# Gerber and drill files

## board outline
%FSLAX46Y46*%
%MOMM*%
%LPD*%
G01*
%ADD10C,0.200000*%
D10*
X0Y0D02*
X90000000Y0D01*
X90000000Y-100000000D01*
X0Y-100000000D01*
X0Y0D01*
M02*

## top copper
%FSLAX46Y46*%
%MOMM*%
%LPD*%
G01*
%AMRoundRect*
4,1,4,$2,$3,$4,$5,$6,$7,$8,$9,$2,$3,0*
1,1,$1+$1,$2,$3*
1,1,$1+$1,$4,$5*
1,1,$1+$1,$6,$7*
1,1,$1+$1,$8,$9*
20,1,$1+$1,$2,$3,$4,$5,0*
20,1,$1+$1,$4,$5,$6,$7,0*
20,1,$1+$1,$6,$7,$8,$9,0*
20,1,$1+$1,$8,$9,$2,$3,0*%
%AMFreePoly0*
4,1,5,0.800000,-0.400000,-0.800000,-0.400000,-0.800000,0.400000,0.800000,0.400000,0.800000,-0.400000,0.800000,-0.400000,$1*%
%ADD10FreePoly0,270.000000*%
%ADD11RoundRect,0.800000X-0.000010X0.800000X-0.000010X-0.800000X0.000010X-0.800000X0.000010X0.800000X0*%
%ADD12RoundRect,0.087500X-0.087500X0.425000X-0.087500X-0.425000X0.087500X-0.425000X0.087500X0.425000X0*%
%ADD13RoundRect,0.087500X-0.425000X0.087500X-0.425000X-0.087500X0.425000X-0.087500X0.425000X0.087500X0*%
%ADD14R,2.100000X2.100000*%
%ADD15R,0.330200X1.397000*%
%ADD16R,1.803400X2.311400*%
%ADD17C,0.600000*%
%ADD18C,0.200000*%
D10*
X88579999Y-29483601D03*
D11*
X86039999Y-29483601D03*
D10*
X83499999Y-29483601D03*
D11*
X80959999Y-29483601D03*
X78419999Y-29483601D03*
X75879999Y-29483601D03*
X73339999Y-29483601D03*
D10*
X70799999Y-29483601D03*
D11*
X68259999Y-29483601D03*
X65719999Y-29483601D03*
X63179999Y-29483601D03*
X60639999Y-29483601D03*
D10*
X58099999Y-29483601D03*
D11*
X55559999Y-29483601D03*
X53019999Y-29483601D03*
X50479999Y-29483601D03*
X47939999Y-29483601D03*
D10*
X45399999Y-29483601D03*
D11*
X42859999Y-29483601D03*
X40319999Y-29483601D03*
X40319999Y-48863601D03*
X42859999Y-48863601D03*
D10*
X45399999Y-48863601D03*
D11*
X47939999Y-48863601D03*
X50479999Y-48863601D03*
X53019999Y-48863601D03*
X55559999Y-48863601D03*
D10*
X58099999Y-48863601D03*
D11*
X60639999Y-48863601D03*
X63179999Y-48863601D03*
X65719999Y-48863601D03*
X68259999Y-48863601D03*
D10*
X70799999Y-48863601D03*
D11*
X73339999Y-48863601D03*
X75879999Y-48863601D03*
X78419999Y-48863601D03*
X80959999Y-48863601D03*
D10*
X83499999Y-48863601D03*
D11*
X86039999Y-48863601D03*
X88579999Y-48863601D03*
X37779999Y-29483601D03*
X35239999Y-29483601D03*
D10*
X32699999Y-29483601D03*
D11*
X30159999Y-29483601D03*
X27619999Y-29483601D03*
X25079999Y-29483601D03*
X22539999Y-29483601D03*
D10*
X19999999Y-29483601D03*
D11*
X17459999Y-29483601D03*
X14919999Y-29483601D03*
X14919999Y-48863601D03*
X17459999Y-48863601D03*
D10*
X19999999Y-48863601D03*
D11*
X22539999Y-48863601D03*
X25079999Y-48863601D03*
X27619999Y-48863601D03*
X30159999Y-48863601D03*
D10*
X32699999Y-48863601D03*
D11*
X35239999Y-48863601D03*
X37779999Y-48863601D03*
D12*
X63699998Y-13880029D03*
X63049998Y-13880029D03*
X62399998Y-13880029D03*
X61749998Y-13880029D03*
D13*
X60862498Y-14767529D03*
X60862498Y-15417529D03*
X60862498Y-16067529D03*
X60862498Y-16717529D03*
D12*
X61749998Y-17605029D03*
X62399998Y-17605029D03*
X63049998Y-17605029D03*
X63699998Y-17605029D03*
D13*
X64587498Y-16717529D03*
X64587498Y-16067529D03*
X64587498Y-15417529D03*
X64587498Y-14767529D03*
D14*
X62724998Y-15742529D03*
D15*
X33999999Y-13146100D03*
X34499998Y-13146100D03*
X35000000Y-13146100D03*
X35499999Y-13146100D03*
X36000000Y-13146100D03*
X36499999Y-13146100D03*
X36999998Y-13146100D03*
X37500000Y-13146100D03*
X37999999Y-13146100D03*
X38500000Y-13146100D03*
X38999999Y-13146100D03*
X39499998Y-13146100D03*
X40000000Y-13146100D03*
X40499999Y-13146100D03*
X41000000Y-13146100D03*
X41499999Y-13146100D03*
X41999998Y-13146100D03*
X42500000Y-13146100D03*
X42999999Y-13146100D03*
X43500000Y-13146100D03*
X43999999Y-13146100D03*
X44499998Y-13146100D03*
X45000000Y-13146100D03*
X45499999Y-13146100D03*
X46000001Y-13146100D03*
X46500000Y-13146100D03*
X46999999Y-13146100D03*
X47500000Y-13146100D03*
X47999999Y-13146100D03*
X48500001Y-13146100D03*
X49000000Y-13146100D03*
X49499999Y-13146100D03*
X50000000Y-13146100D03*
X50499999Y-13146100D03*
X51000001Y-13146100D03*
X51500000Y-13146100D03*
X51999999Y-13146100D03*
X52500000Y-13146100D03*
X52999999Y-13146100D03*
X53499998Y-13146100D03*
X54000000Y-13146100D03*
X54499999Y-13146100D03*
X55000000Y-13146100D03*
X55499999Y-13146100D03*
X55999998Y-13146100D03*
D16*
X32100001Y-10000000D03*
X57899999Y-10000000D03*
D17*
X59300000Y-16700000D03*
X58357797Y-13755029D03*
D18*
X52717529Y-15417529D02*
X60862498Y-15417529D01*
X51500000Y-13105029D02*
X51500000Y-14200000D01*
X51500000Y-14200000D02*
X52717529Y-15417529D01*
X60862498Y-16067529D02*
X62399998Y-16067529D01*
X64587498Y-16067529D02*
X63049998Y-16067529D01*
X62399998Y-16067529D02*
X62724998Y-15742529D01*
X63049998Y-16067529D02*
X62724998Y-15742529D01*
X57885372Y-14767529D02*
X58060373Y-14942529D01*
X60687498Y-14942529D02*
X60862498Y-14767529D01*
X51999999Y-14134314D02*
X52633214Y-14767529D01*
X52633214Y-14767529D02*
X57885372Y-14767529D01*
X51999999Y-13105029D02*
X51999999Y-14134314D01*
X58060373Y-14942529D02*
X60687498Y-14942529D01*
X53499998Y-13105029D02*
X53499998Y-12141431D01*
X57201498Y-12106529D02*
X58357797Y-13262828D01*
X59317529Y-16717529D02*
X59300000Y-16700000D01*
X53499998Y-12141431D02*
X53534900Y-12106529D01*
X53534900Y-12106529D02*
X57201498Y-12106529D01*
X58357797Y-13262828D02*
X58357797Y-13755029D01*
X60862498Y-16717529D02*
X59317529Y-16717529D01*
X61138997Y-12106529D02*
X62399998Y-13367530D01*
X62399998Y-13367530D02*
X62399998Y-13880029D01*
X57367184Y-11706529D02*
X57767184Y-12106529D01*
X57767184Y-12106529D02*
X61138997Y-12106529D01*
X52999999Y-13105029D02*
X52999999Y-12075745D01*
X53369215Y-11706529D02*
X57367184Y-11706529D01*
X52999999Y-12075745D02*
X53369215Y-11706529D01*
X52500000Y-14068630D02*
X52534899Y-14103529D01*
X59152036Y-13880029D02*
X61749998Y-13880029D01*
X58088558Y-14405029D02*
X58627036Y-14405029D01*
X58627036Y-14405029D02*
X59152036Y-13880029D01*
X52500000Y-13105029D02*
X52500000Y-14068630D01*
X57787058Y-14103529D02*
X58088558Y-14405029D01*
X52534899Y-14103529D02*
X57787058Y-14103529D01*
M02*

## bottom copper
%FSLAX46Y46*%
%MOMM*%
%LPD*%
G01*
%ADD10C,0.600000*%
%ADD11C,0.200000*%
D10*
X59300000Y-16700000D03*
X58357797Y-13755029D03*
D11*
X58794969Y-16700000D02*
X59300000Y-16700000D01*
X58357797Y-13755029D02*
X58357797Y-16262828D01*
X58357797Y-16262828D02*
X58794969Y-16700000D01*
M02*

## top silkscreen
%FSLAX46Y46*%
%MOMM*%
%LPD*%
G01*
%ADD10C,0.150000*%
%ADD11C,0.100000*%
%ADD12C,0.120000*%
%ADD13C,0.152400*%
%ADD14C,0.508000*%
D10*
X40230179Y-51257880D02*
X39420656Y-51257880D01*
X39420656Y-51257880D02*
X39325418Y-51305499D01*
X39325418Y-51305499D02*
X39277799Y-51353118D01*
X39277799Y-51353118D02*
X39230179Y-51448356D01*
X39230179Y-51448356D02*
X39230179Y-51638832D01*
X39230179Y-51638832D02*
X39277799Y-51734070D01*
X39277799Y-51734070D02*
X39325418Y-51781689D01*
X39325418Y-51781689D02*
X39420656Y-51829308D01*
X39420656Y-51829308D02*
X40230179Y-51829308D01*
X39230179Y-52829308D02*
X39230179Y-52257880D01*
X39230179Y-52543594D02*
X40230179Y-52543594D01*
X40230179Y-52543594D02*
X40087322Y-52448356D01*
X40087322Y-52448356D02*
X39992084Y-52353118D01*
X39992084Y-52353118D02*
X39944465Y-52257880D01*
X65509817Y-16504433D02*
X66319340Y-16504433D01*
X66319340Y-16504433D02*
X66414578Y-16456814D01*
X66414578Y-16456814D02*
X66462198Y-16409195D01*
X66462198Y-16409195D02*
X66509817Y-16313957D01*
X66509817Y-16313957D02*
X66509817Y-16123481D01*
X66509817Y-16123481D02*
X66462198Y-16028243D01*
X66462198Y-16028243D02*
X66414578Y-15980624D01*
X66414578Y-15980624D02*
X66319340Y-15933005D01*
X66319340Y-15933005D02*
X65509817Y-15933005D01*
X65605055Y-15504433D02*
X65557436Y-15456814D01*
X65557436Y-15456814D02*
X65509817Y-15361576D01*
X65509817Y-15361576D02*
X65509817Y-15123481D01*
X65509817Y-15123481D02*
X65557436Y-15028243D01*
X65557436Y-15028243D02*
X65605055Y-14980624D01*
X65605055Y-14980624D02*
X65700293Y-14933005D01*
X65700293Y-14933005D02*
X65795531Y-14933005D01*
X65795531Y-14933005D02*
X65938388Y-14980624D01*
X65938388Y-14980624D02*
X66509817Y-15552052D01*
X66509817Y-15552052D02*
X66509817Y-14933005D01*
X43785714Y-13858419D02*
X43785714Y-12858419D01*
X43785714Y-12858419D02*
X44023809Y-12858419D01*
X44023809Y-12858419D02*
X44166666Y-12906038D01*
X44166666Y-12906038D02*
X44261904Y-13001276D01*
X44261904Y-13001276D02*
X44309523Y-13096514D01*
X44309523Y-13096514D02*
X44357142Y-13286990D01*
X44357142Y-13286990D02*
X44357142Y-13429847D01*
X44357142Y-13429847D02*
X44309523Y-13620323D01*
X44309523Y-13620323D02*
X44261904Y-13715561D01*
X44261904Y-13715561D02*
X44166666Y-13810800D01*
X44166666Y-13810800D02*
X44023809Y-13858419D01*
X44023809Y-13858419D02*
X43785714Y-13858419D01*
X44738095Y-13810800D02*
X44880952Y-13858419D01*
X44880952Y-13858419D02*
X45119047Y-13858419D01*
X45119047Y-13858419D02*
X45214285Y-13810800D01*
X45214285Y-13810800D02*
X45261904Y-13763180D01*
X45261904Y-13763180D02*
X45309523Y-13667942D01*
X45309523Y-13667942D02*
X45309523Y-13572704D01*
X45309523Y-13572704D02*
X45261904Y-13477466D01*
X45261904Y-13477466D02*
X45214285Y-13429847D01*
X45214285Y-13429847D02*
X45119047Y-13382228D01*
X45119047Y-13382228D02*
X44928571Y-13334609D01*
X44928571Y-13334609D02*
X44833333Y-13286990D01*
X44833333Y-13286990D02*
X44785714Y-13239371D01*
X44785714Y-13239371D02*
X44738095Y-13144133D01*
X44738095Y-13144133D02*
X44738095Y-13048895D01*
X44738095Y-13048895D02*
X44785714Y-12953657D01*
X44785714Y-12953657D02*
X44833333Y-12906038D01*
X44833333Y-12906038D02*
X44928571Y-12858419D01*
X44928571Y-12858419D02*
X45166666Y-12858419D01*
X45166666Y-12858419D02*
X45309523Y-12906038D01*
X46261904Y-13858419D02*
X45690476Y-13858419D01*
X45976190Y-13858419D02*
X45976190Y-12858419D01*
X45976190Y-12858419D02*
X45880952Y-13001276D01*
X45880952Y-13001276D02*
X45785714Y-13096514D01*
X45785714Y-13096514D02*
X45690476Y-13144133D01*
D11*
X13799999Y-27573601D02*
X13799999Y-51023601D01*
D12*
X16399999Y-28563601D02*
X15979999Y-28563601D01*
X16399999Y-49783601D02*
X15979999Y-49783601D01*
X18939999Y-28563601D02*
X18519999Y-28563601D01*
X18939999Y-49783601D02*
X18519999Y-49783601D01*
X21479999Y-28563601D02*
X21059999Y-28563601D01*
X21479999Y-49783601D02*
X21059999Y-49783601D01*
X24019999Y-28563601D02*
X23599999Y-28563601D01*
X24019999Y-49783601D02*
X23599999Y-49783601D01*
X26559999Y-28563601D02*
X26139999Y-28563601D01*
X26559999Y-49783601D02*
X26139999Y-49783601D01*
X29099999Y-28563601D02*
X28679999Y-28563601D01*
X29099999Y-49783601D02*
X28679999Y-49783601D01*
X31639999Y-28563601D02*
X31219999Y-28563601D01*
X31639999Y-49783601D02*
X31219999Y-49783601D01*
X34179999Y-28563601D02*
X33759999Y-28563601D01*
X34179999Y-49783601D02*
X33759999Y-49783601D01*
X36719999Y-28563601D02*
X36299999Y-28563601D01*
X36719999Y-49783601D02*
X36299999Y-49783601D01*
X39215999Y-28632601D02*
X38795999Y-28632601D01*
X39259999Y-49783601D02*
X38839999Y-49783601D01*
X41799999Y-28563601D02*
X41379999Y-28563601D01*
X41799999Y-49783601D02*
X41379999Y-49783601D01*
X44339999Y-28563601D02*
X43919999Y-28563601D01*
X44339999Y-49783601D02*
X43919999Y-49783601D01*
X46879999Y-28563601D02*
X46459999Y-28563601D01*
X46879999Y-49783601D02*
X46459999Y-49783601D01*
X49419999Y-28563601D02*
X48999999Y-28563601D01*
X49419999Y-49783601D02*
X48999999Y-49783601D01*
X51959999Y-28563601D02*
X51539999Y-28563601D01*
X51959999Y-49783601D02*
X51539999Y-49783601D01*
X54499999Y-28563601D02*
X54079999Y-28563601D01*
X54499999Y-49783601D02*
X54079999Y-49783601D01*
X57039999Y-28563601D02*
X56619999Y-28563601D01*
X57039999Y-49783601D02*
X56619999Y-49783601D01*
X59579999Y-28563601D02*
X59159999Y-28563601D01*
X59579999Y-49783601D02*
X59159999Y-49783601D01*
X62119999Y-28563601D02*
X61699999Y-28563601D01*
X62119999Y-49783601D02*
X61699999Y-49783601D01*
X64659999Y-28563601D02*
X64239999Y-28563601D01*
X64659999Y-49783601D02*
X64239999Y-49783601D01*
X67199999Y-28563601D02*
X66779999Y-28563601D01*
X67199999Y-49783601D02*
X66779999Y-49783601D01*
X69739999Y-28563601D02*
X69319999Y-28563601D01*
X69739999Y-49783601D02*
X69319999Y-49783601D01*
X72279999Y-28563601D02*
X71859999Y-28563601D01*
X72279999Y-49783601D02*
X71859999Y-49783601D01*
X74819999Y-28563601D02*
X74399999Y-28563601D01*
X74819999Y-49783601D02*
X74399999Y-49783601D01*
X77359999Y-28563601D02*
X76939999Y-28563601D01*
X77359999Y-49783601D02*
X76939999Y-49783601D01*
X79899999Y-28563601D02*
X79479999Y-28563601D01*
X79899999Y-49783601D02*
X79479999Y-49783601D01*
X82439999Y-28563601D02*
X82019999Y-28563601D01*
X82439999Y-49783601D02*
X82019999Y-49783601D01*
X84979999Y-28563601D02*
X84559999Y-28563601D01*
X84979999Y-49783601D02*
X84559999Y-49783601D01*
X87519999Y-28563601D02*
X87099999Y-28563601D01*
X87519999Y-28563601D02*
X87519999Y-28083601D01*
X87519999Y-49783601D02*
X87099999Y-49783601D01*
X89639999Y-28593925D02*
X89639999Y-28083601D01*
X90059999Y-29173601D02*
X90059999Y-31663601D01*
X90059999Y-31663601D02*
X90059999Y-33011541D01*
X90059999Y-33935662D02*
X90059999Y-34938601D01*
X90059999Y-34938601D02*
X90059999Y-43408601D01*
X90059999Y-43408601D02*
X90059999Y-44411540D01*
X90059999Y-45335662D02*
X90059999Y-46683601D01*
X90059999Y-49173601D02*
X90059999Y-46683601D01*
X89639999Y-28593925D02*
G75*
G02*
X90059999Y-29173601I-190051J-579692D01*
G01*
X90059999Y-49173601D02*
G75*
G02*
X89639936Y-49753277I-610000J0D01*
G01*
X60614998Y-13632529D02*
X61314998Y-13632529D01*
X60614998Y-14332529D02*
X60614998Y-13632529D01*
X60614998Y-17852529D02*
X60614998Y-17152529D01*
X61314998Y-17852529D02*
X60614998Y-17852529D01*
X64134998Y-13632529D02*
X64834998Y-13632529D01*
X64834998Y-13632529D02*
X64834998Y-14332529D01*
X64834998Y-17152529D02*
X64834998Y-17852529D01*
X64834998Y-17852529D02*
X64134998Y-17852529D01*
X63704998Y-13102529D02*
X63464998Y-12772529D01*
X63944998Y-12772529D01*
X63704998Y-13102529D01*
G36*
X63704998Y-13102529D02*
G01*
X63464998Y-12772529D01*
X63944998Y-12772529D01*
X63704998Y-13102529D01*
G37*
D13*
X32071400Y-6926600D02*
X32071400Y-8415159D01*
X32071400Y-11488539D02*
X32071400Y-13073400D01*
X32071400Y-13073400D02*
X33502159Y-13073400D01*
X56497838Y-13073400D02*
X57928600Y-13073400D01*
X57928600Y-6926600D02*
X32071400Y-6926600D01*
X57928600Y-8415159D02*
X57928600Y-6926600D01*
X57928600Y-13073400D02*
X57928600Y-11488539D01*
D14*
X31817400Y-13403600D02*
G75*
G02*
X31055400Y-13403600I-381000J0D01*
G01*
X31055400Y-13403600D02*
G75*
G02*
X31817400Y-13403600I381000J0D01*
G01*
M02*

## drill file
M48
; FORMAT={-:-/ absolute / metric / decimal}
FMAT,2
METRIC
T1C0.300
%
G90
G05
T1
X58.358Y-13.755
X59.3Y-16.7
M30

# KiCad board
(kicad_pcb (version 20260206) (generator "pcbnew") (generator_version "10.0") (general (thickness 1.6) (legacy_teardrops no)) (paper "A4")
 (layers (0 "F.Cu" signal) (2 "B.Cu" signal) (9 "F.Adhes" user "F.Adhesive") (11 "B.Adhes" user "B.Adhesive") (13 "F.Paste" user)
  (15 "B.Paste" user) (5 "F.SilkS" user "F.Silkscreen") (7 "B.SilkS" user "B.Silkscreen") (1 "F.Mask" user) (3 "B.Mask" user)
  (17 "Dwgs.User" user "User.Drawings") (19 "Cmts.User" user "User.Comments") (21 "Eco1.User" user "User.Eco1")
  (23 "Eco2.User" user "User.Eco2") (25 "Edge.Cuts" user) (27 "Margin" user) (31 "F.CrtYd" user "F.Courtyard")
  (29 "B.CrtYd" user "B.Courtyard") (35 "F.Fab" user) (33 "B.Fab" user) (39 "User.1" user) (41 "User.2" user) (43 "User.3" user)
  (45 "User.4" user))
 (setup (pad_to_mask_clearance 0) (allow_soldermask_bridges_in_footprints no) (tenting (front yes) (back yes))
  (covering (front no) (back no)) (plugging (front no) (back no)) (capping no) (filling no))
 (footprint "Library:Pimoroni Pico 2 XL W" (layer "F.Cu") (at 64.449999 39.173601 -90)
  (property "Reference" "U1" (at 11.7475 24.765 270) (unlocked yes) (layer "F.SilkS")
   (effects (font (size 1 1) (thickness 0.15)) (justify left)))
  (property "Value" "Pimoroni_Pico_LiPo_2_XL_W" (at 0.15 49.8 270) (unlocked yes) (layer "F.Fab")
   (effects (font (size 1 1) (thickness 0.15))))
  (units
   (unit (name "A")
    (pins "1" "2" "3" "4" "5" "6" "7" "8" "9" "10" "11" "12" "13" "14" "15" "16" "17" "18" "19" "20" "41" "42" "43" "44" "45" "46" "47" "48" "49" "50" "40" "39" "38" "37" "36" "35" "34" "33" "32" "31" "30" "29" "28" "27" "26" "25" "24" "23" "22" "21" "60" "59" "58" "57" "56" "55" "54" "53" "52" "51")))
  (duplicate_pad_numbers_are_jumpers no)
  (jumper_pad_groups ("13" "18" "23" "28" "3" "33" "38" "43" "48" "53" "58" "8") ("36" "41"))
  (fp_line (start -11.6 50.65) (end 11.85 50.65) (stroke (width 0.1) (type default)) (layer "F.SilkS"))
  (fp_line (start -10.61 48.05) (end -10.61 48.47) (stroke (width 0.12) (type solid)) (layer "F.SilkS"))
  (fp_line (start 10.61 48.05) (end 10.61 48.47) (stroke (width 0.12) (type solid)) (layer "F.SilkS"))
  (fp_line (start -10.61 45.51) (end -10.61 45.93) (stroke (width 0.12) (type solid)) (layer "F.SilkS"))
  (fp_line (start 10.61 45.51) (end 10.61 45.93) (stroke (width 0.12) (type solid)) (layer "F.SilkS"))
  (fp_line (start -10.61 42.97) (end -10.61 43.39) (stroke (width 0.12) (type solid)) (layer "F.SilkS"))
  (fp_line (start 10.61 42.97) (end 10.61 43.39) (stroke (width 0.12) (type solid)) (layer "F.SilkS"))
  (fp_line (start -10.61 40.43) (end -10.61 40.85) (stroke (width 0.12) (type solid)) (layer "F.SilkS"))
  (fp_line (start 10.61 40.43) (end 10.61 40.85) (stroke (width 0.12) (type solid)) (layer "F.SilkS"))
  (fp_line (start -10.61 37.89) (end -10.61 38.31) (stroke (width 0.12) (type solid)) (layer "F.SilkS"))
  (fp_line (start 10.61 37.89) (end 10.61 38.31) (stroke (width 0.12) (type solid)) (layer "F.SilkS"))
  (fp_line (start -10.61 35.35) (end -10.61 35.77) (stroke (width 0.12) (type solid)) (layer "F.SilkS"))
  (fp_line (start 10.61 35.35) (end 10.61 35.77) (stroke (width 0.12) (type solid)) (layer "F.SilkS"))
  (fp_line (start -10.61 32.81) (end -10.61 33.23) (stroke (width 0.12) (type solid)) (layer "F.SilkS"))
  (fp_line (start 10.61 32.81) (end 10.61 33.23) (stroke (width 0.12) (type solid)) (layer "F.SilkS"))
  (fp_line (start -10.61 30.27) (end -10.61 30.69) (stroke (width 0.12) (type solid)) (layer "F.SilkS"))
  (fp_line (start 10.61 30.27) (end 10.61 30.69) (stroke (width 0.12) (type solid)) (layer "F.SilkS"))
  (fp_line (start -10.61 27.73) (end -10.61 28.15) (stroke (width 0.12) (type solid)) (layer "F.SilkS"))
  (fp_line (start 10.61 27.73) (end 10.61 28.15) (stroke (width 0.12) (type solid)) (layer "F.SilkS"))
  (fp_line (start -10.541 25.234) (end -10.541 25.654) (stroke (width 0.12) (type solid)) (layer "F.SilkS"))
  (fp_line (start 10.61 25.19) (end 10.61 25.61) (stroke (width 0.12) (type solid)) (layer "F.SilkS"))
  (fp_line (start -10.61 22.65) (end -10.61 23.07) (stroke (width 0.12) (type solid)) (layer "F.SilkS"))
  (fp_line (start 10.61 22.65) (end 10.61 23.07) (stroke (width 0.12) (type solid)) (layer "F.SilkS"))
  (fp_line (start -10.61 20.11) (end -10.61 20.53) (stroke (width 0.12) (type solid)) (layer "F.SilkS"))
  (fp_line (start 10.61 20.11) (end 10.61 20.53) (stroke (width 0.12) (type solid)) (layer "F.SilkS"))
  (fp_line (start -10.61 17.57) (end -10.61 17.99) (stroke (width 0.12) (type solid)) (layer "F.SilkS"))
  (fp_line (start 10.61 17.57) (end 10.61 17.99) (stroke (width 0.12) (type solid)) (layer "F.SilkS"))
  (fp_line (start -10.61 15.03) (end -10.61 15.45) (stroke (width 0.12) (type solid)) (layer "F.SilkS"))
  (fp_line (start 10.61 15.03) (end 10.61 15.45) (stroke (width 0.12) (type solid)) (layer "F.SilkS"))
  (fp_line (start -10.61 12.49) (end -10.61 12.91) (stroke (width 0.12) (type solid)) (layer "F.SilkS"))
  (fp_line (start 10.61 12.49) (end 10.61 12.91) (stroke (width 0.12) (type solid)) (layer "F.SilkS"))
  (fp_line (start -10.61 9.95) (end -10.61 10.37) (stroke (width 0.12) (type solid)) (layer "F.SilkS"))
  (fp_line (start 10.61 9.95) (end 10.61 10.37) (stroke (width 0.12) (type solid)) (layer "F.SilkS"))
  (fp_line (start -10.61 7.41) (end -10.61 7.83) (stroke (width 0.12) (type solid)) (layer "F.SilkS"))
  (fp_line (start 10.61 7.41) (end 10.61 7.83) (stroke (width 0.12) (type solid)) (layer "F.SilkS"))
  (fp_line (start -10.61 4.87) (end -10.61 5.29) (stroke (width 0.12) (type solid)) (layer "F.SilkS"))
  (fp_line (start 10.61 4.87) (end 10.61 5.29) (stroke (width 0.12) (type solid)) (layer "F.SilkS"))
  (fp_line (start -10.61 2.33) (end -10.61 2.75) (stroke (width 0.12) (type solid)) (layer "F.SilkS"))
  (fp_line (start 10.61 2.33) (end 10.61 2.75) (stroke (width 0.12) (type solid)) (layer "F.SilkS"))
  (fp_line (start -10.61 -0.21) (end -10.61 0.21) (stroke (width 0.12) (type solid)) (layer "F.SilkS"))
  (fp_line (start 10.61 -0.21) (end 10.61 0.21) (stroke (width 0.12) (type solid)) (layer "F.SilkS"))
  (fp_line (start -10.61 -2.75) (end -10.61 -2.33) (stroke (width 0.12) (type solid)) (layer "F.SilkS"))
  (fp_line (start 10.61 -2.75) (end 10.61 -2.33) (stroke (width 0.12) (type solid)) (layer "F.SilkS"))
  (fp_line (start -10.61 -5.29) (end -10.61 -4.87) (stroke (width 0.12) (type solid)) (layer "F.SilkS"))
  (fp_line (start 10.61 -5.29) (end 10.61 -4.87) (stroke (width 0.12) (type solid)) (layer "F.SilkS"))
  (fp_line (start -10.61 -7.83) (end -10.61 -7.41) (stroke (width 0.12) (type solid)) (layer "F.SilkS"))
  (fp_line (start 10.61 -7.83) (end 10.61 -7.41) (stroke (width 0.12) (type solid)) (layer "F.SilkS"))
  (fp_line (start -10.61 -10.37) (end -10.61 -9.95) (stroke (width 0.12) (type solid)) (layer "F.SilkS"))
  (fp_line (start 10.61 -10.37) (end 10.61 -9.95) (stroke (width 0.12) (type solid)) (layer "F.SilkS"))
  (fp_line (start -10.61 -12.91) (end -10.61 -12.49) (stroke (width 0.12) (type solid)) (layer "F.SilkS"))
  (fp_line (start 10.61 -12.91) (end 10.61 -12.49) (stroke (width 0.12) (type solid)) (layer "F.SilkS"))
  (fp_line (start -10.61 -15.45) (end -10.61 -15.03) (stroke (width 0.12) (type solid)) (layer "F.SilkS"))
  (fp_line (start 10.61 -15.45) (end 10.61 -15.03) (stroke (width 0.12) (type solid)) (layer "F.SilkS"))
  (fp_line (start -10.61 -17.99) (end -10.61 -17.57) (stroke (width 0.12) (type solid)) (layer "F.SilkS"))
  (fp_line (start 10.61 -17.99) (end 10.61 -17.57) (stroke (width 0.12) (type solid)) (layer "F.SilkS"))
  (fp_line (start -10.61 -20.53) (end -10.61 -20.11) (stroke (width 0.12) (type solid)) (layer "F.SilkS"))
  (fp_line (start 10.61 -20.53) (end 10.61 -20.11) (stroke (width 0.12) (type solid)) (layer "F.SilkS"))
  (fp_line (start -10.61 -23.07) (end -10.61 -22.65) (stroke (width 0.12) (type solid)) (layer "F.SilkS"))
  (fp_line (start -10.61 -23.07) (end -11.09 -23.07) (stroke (width 0.12) (type solid)) (layer "F.SilkS"))
  (fp_line (start 10.61 -23.07) (end 10.61 -22.65) (stroke (width 0.12) (type solid)) (layer "F.SilkS"))
  (fp_line (start -10.579676 -25.19) (end -11.09 -25.19) (stroke (width 0.12) (type solid)) (layer "F.SilkS"))
  (fp_line (start -10 -25.61) (end -7.51 -25.61) (stroke (width 0.12) (type solid)) (layer "F.SilkS"))
  (fp_line (start -7.51 -25.61) (end -6.16206 -25.61) (stroke (width 0.12) (type solid)) (layer "F.SilkS"))
  (fp_line (start -5.237939 -25.61) (end -4.235 -25.61) (stroke (width 0.12) (type solid)) (layer "F.SilkS"))
  (fp_line (start -4.235 -25.61) (end 4.235 -25.61) (stroke (width 0.12) (type solid)) (layer "F.SilkS"))
  (fp_line (start 4.235 -25.61) (end 5.237939 -25.61) (stroke (width 0.12) (type solid)) (layer "F.SilkS"))
  (fp_line (start 6.162061 -25.61) (end 7.51 -25.61) (stroke (width 0.12) (type solid)) (layer "F.SilkS"))
  (fp_line (start 10 -25.61) (end 7.51 -25.61) (stroke (width 0.12) (type solid)) (layer "F.SilkS"))
  (fp_arc (start -10.579676 -25.19) (mid -10.357938 -25.493944) (end -10 -25.61) (stroke (width 0.12) (type solid)) (layer "F.SilkS"))
  (fp_arc (start 10 -25.61) (mid 10.357937 -25.493944) (end 10.579676 -25.189937) (stroke (width 0.12) (type solid)) (layer "F.SilkS"))
  (pad "" smd rect (at -8.89 -24.13 270) (size 3.8 2.2) (drill (offset -0.8 0)) (layers "F.Paste"))
  (pad "" smd rect (at -8.89 -21.59 270) (size 3.8 2.2) (drill (offset -0.8 0)) (layers "F.Paste"))
  (pad "" smd rect (at -8.89 -19.05 270) (size 3.8 2.2) (drill (offset -0.8 0)) (layers "F.Paste"))
  (pad "" smd rect (at -8.89 -16.51 270) (size 3.8 2.2) (drill (offset -0.8 0)) (layers "F.Paste"))
  (pad "" smd rect (at -8.89 -13.97 270) (size 3.8 2.2) (drill (offset -0.8 0)) (layers "F.Paste"))
  (pad "" smd rect (at -8.89 -11.43 270) (size 3.8 2.2) (drill (offset -0.8 0)) (layers "F.Paste"))
  (pad "" smd rect (at -8.89 -8.89 270) (size 3.8 2.2) (drill (offset -0.8 0)) (layers "F.Paste"))
  (pad "" smd rect (at -8.89 -6.35 270) (size 3.8 2.2) (drill (offset -0.8 0)) (layers "F.Paste"))
  (pad "" smd rect (at -8.89 -3.81 270) (size 3.8 2.2) (drill (offset -0.8 0)) (layers "F.Paste"))
  (pad "" smd rect (at -8.89 -1.27 270) (size 3.8 2.2) (drill (offset -0.8 0)) (layers "F.Paste"))
  (pad "" smd rect (at -8.89 1.27 270) (size 3.8 2.2) (drill (offset -0.8 0)) (layers "F.Paste"))
  (pad "" smd rect (at -8.89 3.81 270) (size 3.8 2.2) (drill (offset -0.8 0)) (layers "F.Paste"))
  (pad "" smd rect (at -8.89 6.35 270) (size 3.8 2.2) (drill (offset -0.8 0)) (layers "F.Paste"))
  (pad "" smd rect (at -8.89 8.89 270) (size 3.8 2.2) (drill (offset -0.8 0)) (layers "F.Paste"))
  (pad "" smd rect (at -8.89 11.43 270) (size 3.8 2.2) (drill (offset -0.8 0)) (layers "F.Paste"))
  (pad "" smd rect (at -8.89 13.97 270) (size 3.8 2.2) (drill (offset -0.8 0)) (layers "F.Paste"))
  (pad "" smd rect (at -8.89 16.51 270) (size 3.8 2.2) (drill (offset -0.8 0)) (layers "F.Paste"))
  (pad "" smd rect (at -8.89 19.05 270) (size 3.8 2.2) (drill (offset -0.8 0)) (layers "F.Paste"))
  (pad "" smd rect (at -8.89 21.59 270) (size 3.8 2.2) (drill (offset -0.8 0)) (layers "F.Paste"))
  (pad "" smd rect (at -8.89 24.13 270) (size 3.8 2.2) (drill (offset -0.8 0)) (layers "F.Paste"))
  (pad "" smd rect (at -8.89 26.67 270) (size 3.8 2.2) (drill (offset -0.8 0)) (layers "F.Paste"))
  (pad "" smd rect (at -8.89 29.21 270) (size 3.8 2.2) (drill (offset -0.8 0)) (layers "F.Paste"))
  (pad "" smd rect (at -8.89 31.75 270) (size 3.8 2.2) (drill (offset -0.8 0)) (layers "F.Paste"))
  (pad "" smd rect (at -8.89 34.29 270) (size 3.8 2.2) (drill (offset -0.8 0)) (layers "F.Paste"))
  (pad "" smd rect (at -8.89 36.83 270) (size 3.8 2.2) (drill (offset -0.8 0)) (layers "F.Paste"))
  (pad "" smd rect (at -8.89 39.37 270) (size 3.8 2.2) (drill (offset -0.8 0)) (layers "F.Paste"))
  (pad "" smd rect (at -8.89 41.91 270) (size 3.8 2.2) (drill (offset -0.8 0)) (layers "F.Paste"))
  (pad "" smd rect (at -8.89 44.45 270) (size 3.8 2.2) (drill (offset -0.8 0)) (layers "F.Paste"))
  (pad "" smd rect (at -8.89 46.99 270) (size 3.8 2.2) (drill (offset -0.8 0)) (layers "F.Paste"))
  (pad "" smd rect (at -8.89 49.53 270) (size 3.8 2.2) (drill (offset -0.8 0)) (layers "F.Paste"))
  (pad "" smd rect (at 8.89 -24.13 270) (size 3.8 2.2) (drill (offset 0.8 0)) (layers "F.Paste"))
  (pad "" smd rect (at 8.89 -21.59 270) (size 3.8 2.2) (drill (offset 0.8 0)) (layers "F.Paste"))
  (pad "" smd rect (at 8.89 -19.05 270) (size 3.8 2.2) (drill (offset 0.8 0)) (layers "F.Paste"))
  (pad "" smd rect (at 8.89 -16.51 270) (size 3.8 2.2) (drill (offset 0.8 0)) (layers "F.Paste"))
  (pad "" smd rect (at 8.89 -13.97 270) (size 3.8 2.2) (drill (offset 0.8 0)) (layers "F.Paste"))
  (pad "" smd rect (at 8.89 -11.43 270) (size 3.8 2.2) (drill (offset 0.8 0)) (layers "F.Paste"))
  (pad "" smd rect (at 8.89 -8.89 270) (size 3.8 2.2) (drill (offset 0.8 0)) (layers "F.Paste"))
  (pad "" smd rect (at 8.89 -6.35 270) (size 3.8 2.2) (drill (offset 0.8 0)) (layers "F.Paste"))
  (pad "" smd rect (at 8.89 -3.81 270) (size 3.8 2.2) (drill (offset 0.8 0)) (layers "F.Paste"))
  (pad "" smd rect (at 8.89 -1.27 270) (size 3.8 2.2) (drill (offset 0.8 0)) (layers "F.Paste"))
  (pad "" smd rect (at 8.89 1.27 270) (size 3.8 2.2) (drill (offset 0.8 0)) (layers "F.Paste"))
  (pad "" smd rect (at 8.89 3.81 270) (size 3.8 2.2) (drill (offset 0.8 0)) (layers "F.Paste"))
  (pad "" smd rect (at 8.89 6.35 270) (size 3.8 2.2) (drill (offset 0.8 0)) (layers "F.Paste"))
  (pad "" smd rect (at 8.89 8.89 270) (size 3.8 2.2) (drill (offset 0.8 0)) (layers "F.Paste"))
  (pad "" smd rect (at 8.89 11.43 270) (size 3.8 2.2) (drill (offset 0.8 0)) (layers "F.Paste"))
  (pad "" smd rect (at 8.89 13.97 270) (size 3.8 2.2) (drill (offset 0.8 0)) (layers "F.Paste"))
  (pad "" smd rect (at 8.89 16.51 270) (size 3.8 2.2) (drill (offset 0.8 0)) (layers "F.Paste"))
  (pad "" smd rect (at 8.89 19.05 270) (size 3.8 2.2) (drill (offset 0.8 0)) (layers "F.Paste"))
  (pad "" smd rect (at 8.89 21.59 270) (size 3.8 2.2) (drill (offset 0.8 0)) (layers "F.Paste"))
  (pad "" smd rect (at 8.89 24.13 270) (size 3.8 2.2) (drill (offset 0.8 0)) (layers "F.Paste"))
  (pad "" smd rect (at 8.89 26.67 270) (size 3.8 2.2) (drill (offset 0.8 0)) (layers "F.Paste"))
  (pad "" smd rect (at 8.89 29.21 270) (size 3.8 2.2) (drill (offset 0.8 0)) (layers "F.Paste"))
  (pad "" smd rect (at 8.89 31.75 270) (size 3.8 2.2) (drill (offset 0.8 0)) (layers "F.Paste"))
  (pad "" smd rect (at 8.89 34.29 270) (size 3.8 2.2) (drill (offset 0.8 0)) (layers "F.Paste"))
  (pad "" smd rect (at 8.89 36.83 270) (size 3.8 2.2) (drill (offset 0.8 0)) (layers "F.Paste"))
  (pad "" smd rect (at 8.89 39.37 270) (size 3.8 2.2) (drill (offset 0.8 0)) (layers "F.Paste"))
  (pad "" smd rect (at 8.89 41.91 270) (size 3.8 2.2) (drill (offset 0.8 0)) (layers "F.Paste"))
  (pad "" smd rect (at 8.89 44.45 270) (size 3.8 2.2) (drill (offset 0.8 0)) (layers "F.Paste"))
  (pad "" smd rect (at 8.89 46.99 270) (size 3.8 2.2) (drill (offset 0.8 0)) (layers "F.Paste"))
  (pad "" smd rect (at 8.89 49.53 270) (size 3.8 2.2) (drill (offset 0.8 0)) (layers "F.Paste"))
  (pad "1" smd custom (at -9.69 -24.13 270) (size 1.6 0.8) (layers "F.Cu" "F.Mask") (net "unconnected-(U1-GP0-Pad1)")
   (options (clearance outline) (anchor rect)) (primitives))
  (pad "2" smd roundrect (at -9.69 -21.59 270) (size 3.2 1.6) (layers "F.Cu" "F.Mask") (roundrect_rratio 0.5)
   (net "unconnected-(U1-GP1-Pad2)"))
  (pad "3" smd custom (at -9.69 -19.05 270) (size 1.6 0.8) (layers "F.Cu" "F.Mask") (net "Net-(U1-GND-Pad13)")
   (options (clearance outline) (anchor rect)) (primitives))
  (pad "4" smd roundrect (at -9.69 -16.51 270) (size 3.2 1.6) (layers "F.Cu" "F.Mask") (roundrect_rratio 0.5)
   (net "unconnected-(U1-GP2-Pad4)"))
  (pad "5" smd roundrect (at -9.69 -13.97 270) (size 3.2 1.6) (layers "F.Cu" "F.Mask") (roundrect_rratio 0.5)
   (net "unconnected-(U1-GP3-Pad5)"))
  (pad "6" smd roundrect (at -9.69 -11.43 270) (size 3.2 1.6) (layers "F.Cu" "F.Mask") (roundrect_rratio 0.5)
   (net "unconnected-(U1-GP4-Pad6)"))
  (pad "7" smd roundrect (at -9.69 -8.89 270) (size 3.2 1.6) (layers "F.Cu" "F.Mask") (roundrect_rratio 0.5)
   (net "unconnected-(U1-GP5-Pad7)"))
  (pad "8" smd custom (at -9.69 -6.35 270) (size 1.6 0.8) (layers "F.Cu" "F.Mask") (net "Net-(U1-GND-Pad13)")
   (options (clearance outline) (anchor rect)) (primitives))
  (pad "9" smd roundrect (at -9.69 -3.81 270) (size 3.2 1.6) (layers "F.Cu" "F.Mask") (roundrect_rratio 0.5)
   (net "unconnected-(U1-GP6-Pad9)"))
  (pad "10" smd roundrect (at -9.69 -1.27 270) (size 3.2 1.6) (layers "F.Cu" "F.Mask") (roundrect_rratio 0.5)
   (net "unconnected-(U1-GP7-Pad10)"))
  (pad "11" smd roundrect (at -9.69 1.27 270) (size 3.2 1.6) (layers "F.Cu" "F.Mask") (roundrect_rratio 0.5) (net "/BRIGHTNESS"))
  (pad "12" smd roundrect (at -9.69 3.81 270) (size 3.2 1.6) (layers "F.Cu" "F.Mask") (roundrect_rratio 0.5) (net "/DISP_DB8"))
  (pad "13" smd custom (at -9.69 6.35 270) (size 1.6 0.8) (layers "F.Cu" "F.Mask") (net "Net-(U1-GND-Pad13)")
   (options (clearance outline) (anchor rect)) (primitives))
  (pad "14" smd roundrect (at -9.69 8.89 270) (size 3.2 1.6) (layers "F.Cu" "F.Mask") (roundrect_rratio 0.5) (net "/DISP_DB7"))
  (pad "15" smd roundrect (at -9.69 11.43 270) (size 3.2 1.6) (layers "F.Cu" "F.Mask") (roundrect_rratio 0.5) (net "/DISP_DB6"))
  (pad "16" smd roundrect (at -9.69 13.97 270) (size 3.2 1.6) (layers "F.Cu" "F.Mask") (roundrect_rratio 0.5) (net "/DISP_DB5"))
  (pad "17" smd roundrect (at -9.69 16.51 270) (size 3.2 1.6) (layers "F.Cu" "F.Mask") (roundrect_rratio 0.5) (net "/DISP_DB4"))
  (pad "18" smd custom (at -9.69 19.05 270) (size 1.6 0.8) (layers "F.Cu" "F.Mask") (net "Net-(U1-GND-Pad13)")
   (options (clearance outline) (anchor rect)) (primitives))
  (pad "19" smd roundrect (at -9.69 21.59 270) (size 3.2 1.6) (layers "F.Cu" "F.Mask") (roundrect_rratio 0.5) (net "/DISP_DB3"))
  (pad "20" smd roundrect (at -9.69 24.13 270) (size 3.2 1.6) (layers "F.Cu" "F.Mask") (roundrect_rratio 0.5) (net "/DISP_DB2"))
  (pad "21" smd roundrect (at 9.69 24.13 270) (size 3.2 1.6) (layers "F.Cu" "F.Mask") (roundrect_rratio 0.5)
   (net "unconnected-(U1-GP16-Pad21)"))
  (pad "22" smd roundrect (at 9.69 21.59 270) (size 3.2 1.6) (layers "F.Cu" "F.Mask") (roundrect_rratio 0.5)
   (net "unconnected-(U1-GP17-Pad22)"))
  (pad "23" smd custom (at 9.69 19.05 270) (size 1.6 0.8) (layers "F.Cu" "F.Mask") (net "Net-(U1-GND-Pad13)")
   (options (clearance outline) (anchor rect)) (primitives))
  (pad "24" smd roundrect (at 9.69 16.51 270) (size 3.2 1.6) (layers "F.Cu" "F.Mask") (roundrect_rratio 0.5)
   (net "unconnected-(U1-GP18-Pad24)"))
  (pad "25" smd roundrect (at 9.69 13.97 270) (size 3.2 1.6) (layers "F.Cu" "F.Mask") (roundrect_rratio 0.5)
   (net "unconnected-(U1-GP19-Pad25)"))
  (pad "26" smd roundrect (at 9.69 11.43 270) (size 3.2 1.6) (layers "F.Cu" "F.Mask") (roundrect_rratio 0.5)
   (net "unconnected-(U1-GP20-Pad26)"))
  (pad "27" smd roundrect (at 9.69 8.89 270) (size 3.2 1.6) (layers "F.Cu" "F.Mask") (roundrect_rratio 0.5)
   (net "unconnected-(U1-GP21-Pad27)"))
  (pad "28" smd custom (at 9.69 6.35 270) (size 1.6 0.8) (layers "F.Cu" "F.Mask") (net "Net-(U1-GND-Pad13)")
   (options (clearance outline) (anchor rect)) (primitives))
  (pad "29" smd roundrect (at 9.69 3.81 270) (size 3.2 1.6) (layers "F.Cu" "F.Mask") (roundrect_rratio 0.5)
   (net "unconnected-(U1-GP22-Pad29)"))
  (pad "30" smd roundrect (at 9.69 1.27 270) (size 3.2 1.6) (layers "F.Cu" "F.Mask") (roundrect_rratio 0.5)
   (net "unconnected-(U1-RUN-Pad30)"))
  (pad "31" smd roundrect (at 9.69 -1.27 270) (size 3.2 1.6) (layers "F.Cu" "F.Mask") (roundrect_rratio 0.5)
   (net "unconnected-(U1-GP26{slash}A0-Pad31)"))
  (pad "32" smd roundrect (at 9.69 -3.81 270) (size 3.2 1.6) (layers "F.Cu" "F.Mask") (roundrect_rratio 0.5)
   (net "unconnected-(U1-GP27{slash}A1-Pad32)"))
  (pad "33" smd custom (at 9.69 -6.35 270) (size 1.6 0.8) (layers "F.Cu" "F.Mask") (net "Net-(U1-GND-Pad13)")
   (options (clearance outline) (anchor rect)) (primitives))
  (pad "34" smd roundrect (at 9.69 -8.89 270) (size 3.2 1.6) (layers "F.Cu" "F.Mask") (roundrect_rratio 0.5)
   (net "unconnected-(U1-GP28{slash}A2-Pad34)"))
  (pad "35" smd roundrect (at 9.69 -11.43 270) (size 3.2 1.6) (layers "F.Cu" "F.Mask") (roundrect_rratio 0.5)
   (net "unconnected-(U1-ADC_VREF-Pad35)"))
  (pad "36" smd roundrect (at 9.69 -13.97 270) (size 3.2 1.6) (layers "F.Cu" "F.Mask") (roundrect_rratio 0.5) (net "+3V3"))
  (pad "37" smd roundrect (at 9.69 -16.51 270) (size 3.2 1.6) (layers "F.Cu" "F.Mask") (roundrect_rratio 0.5)
   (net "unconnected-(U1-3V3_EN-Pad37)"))
  (pad "38" smd custom (at 9.69 -19.05 270) (size 1.6 0.8) (layers "F.Cu" "F.Mask") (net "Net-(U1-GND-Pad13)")
   (options (clearance outline) (anchor rect)) (primitives))
  (pad "39" smd roundrect (at 9.69 -21.59 270) (size 3.2 1.6) (layers "F.Cu" "F.Mask") (roundrect_rratio 0.5)
   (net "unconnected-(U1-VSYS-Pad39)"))
  (pad "40" smd roundrect (at 9.69 -24.13 270) (size 3.2 1.6) (layers "F.Cu" "F.Mask") (roundrect_rratio 0.5)
   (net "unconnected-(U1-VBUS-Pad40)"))
  (pad "41" smd roundrect (at -9.69 26.67 270) (size 3.2 1.6) (layers "F.Cu" "F.Mask") (roundrect_rratio 0.5) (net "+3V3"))
  (pad "42" smd roundrect (at -9.69 29.21 270) (size 3.2 1.6) (layers "F.Cu" "F.Mask") (roundrect_rratio 0.5) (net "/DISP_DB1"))
  (pad "43" smd custom (at -9.69 31.75 270) (size 1.6 0.8) (layers "F.Cu" "F.Mask") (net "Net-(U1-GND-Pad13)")
   (options (clearance outline) (anchor rect)) (primitives))
  (pad "44" smd roundrect (at -9.69 34.29 270) (size 3.2 1.6) (layers "F.Cu" "F.Mask") (roundrect_rratio 0.5) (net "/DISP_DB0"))
  (pad "45" smd roundrect (at -9.69 36.83 270) (size 3.2 1.6) (layers "F.Cu" "F.Mask") (roundrect_rratio 0.5) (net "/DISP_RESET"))
  (pad "46" smd roundrect (at -9.69 39.37 270) (size 3.2 1.6) (layers "F.Cu" "F.Mask") (roundrect_rratio 0.5) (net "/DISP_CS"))
  (pad "47" smd roundrect (at -9.69 41.91 270) (size 3.2 1.6) (layers "F.Cu" "F.Mask") (roundrect_rratio 0.5) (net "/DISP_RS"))
  (pad "48" smd custom (at -9.69 44.45 270) (size 1.6 0.8) (layers "F.Cu" "F.Mask") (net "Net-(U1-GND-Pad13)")
   (options (clearance outline) (anchor rect)) (primitives))
  (pad "49" smd roundrect (at -9.69 46.99 270) (size 3.2 1.6) (layers "F.Cu" "F.Mask") (roundrect_rratio 0.5) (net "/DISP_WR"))
  (pad "50" smd roundrect (at -9.69 49.53 270) (size 3.2 1.6) (layers "F.Cu" "F.Mask") (roundrect_rratio 0.5) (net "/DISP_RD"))
  (pad "51" smd roundrect (at 9.69 49.53 270) (size 3.2 1.6) (layers "F.Cu" "F.Mask") (roundrect_rratio 0.5)
   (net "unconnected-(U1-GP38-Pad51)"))
  (pad "52" smd roundrect (at 9.69 46.99 270) (size 3.2 1.6) (layers "F.Cu" "F.Mask") (roundrect_rratio 0.5)
   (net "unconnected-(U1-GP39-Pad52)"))
  (pad "53" smd custom (at 9.69 44.45 270) (size 1.6 0.8) (layers "F.Cu" "F.Mask") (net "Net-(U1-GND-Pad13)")
   (options (clearance outline) (anchor rect)) (primitives))
  (pad "54" smd roundrect (at 9.69 41.91 270) (size 3.2 1.6) (layers "F.Cu" "F.Mask") (roundrect_rratio 0.5)
   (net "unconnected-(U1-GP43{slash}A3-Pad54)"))
  (pad "55" smd roundrect (at 9.69 39.37 270) (size 3.2 1.6) (layers "F.Cu" "F.Mask") (roundrect_rratio 0.5)
   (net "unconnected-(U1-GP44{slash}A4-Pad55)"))
  (pad "56" smd roundrect (at 9.69 36.83 270) (size 3.2 1.6) (layers "F.Cu" "F.Mask") (roundrect_rratio 0.5)
   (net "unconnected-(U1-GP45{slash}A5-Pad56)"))
  (pad "57" smd roundrect (at 9.69 34.29 270) (size 3.2 1.6) (layers "F.Cu" "F.Mask") (roundrect_rratio 0.5)
   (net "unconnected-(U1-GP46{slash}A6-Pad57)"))
  (pad "58" smd custom (at 9.69 31.75 270) (size 1.6 0.8) (layers "F.Cu" "F.Mask") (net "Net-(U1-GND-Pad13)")
   (options (clearance outline) (anchor rect)) (primitives))
  (pad "59" smd roundrect (at 9.69 29.21 270) (size 3.2 1.6) (layers "F.Cu" "F.Mask") (roundrect_rratio 0.5)
   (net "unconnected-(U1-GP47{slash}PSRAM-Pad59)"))
  (pad "60" smd roundrect (at 9.69 26.67 270) (size 3.2 1.6) (layers "F.Cu" "F.Mask") (roundrect_rratio 0.5)
   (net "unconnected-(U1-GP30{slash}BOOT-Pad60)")))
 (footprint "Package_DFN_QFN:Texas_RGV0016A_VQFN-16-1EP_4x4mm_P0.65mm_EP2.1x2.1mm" (layer "F.Cu") (at 62.724998 15.742529 -90)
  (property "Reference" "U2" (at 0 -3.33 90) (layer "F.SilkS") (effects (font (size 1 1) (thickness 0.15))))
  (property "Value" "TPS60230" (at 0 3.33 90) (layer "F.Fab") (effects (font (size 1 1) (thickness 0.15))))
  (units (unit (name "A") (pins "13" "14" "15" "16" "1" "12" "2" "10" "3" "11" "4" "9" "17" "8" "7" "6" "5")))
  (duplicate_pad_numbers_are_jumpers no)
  (fp_line (start -2.11 2.11) (end -2.11 1.41) (stroke (width 0.12) (type solid)) (layer "F.SilkS"))
  (fp_line (start -1.41 2.11) (end -2.11 2.11) (stroke (width 0.12) (type solid)) (layer "F.SilkS"))
  (fp_line (start 2.11 2.11) (end 1.41 2.11) (stroke (width 0.12) (type solid)) (layer "F.SilkS"))
  (fp_line (start 2.11 1.41) (end 2.11 2.11) (stroke (width 0.12) (type solid)) (layer "F.SilkS"))
  (fp_line (start -2.11 -1.41) (end -2.11 -2.11) (stroke (width 0.12) (type solid)) (layer "F.SilkS"))
  (fp_line (start -2.11 -2.11) (end -1.41 -2.11) (stroke (width 0.12) (type solid)) (layer "F.SilkS"))
  (fp_line (start 1.41 -2.11) (end 2.11 -2.11) (stroke (width 0.12) (type solid)) (layer "F.SilkS"))
  (fp_line (start 2.11 -2.11) (end 2.11 -1.41) (stroke (width 0.12) (type solid)) (layer "F.SilkS"))
  (fp_poly (pts (xy -2.64 -0.98) (xy -2.97 -0.74) (xy -2.97 -1.22)) (stroke (width 0.12) (type solid)) (fill yes) (layer "F.SilkS"))
  (pad "" smd roundrect (at -0.525 -0.525 270) (size 0.85 0.85) (layers "F.Paste") (roundrect_rratio 0.25))
  (pad "" smd roundrect (at -0.525 0.525 270) (size 0.85 0.85) (layers "F.Paste") (roundrect_rratio 0.25))
  (pad "" smd roundrect (at 0.525 -0.525 270) (size 0.85 0.85) (layers "F.Paste") (roundrect_rratio 0.25))
  (pad "" smd roundrect (at 0.525 0.525 270) (size 0.85 0.85) (layers "F.Paste") (roundrect_rratio 0.25))
  (pad "1" smd roundrect (at -1.8625 -0.975 270) (size 1.025 0.35) (layers "F.Cu" "F.Mask" "F.Paste") (roundrect_rratio 0.25)
   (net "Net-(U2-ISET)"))
  (pad "2" smd roundrect (at -1.8625 -0.325 270) (size 1.025 0.35) (layers "F.Cu" "F.Mask" "F.Paste") (roundrect_rratio 0.25)
   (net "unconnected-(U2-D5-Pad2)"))
  (pad "3" smd roundrect (at -1.8625 0.325 270) (size 1.025 0.35) (layers "F.Cu" "F.Mask" "F.Paste") (roundrect_rratio 0.25) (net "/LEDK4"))
  (pad "4" smd roundrect (at -1.8625 0.975 270) (size 1.025 0.35) (layers "F.Cu" "F.Mask" "F.Paste") (roundrect_rratio 0.25) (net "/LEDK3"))
  (pad "5" smd roundrect (at -0.975 1.8625 270) (size 0.35 1.025) (layers "F.Cu" "F.Mask" "F.Paste") (roundrect_rratio 0.25) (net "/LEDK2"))
  (pad "6" smd roundrect (at -0.325 1.8625 270) (size 0.35 1.025) (layers "F.Cu" "F.Mask" "F.Paste") (roundrect_rratio 0.25) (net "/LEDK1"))
  (pad "7" smd roundrect (at 0.325 1.8625 270) (size 0.35 1.025) (layers "F.Cu" "F.Mask" "F.Paste") (roundrect_rratio 0.25) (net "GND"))
  (pad "8" smd roundrect (at 0.975 1.8625 270) (size 0.35 1.025) (layers "F.Cu" "F.Mask" "F.Paste") (roundrect_rratio 0.25) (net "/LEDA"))
  (pad "9" smd roundrect (at 1.8625 0.975 270) (size 1.025 0.35) (layers "F.Cu" "F.Mask" "F.Paste") (roundrect_rratio 0.25)
   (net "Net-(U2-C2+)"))
  (pad "10" smd roundrect (at 1.8625 0.325 270) (size 1.025 0.35) (layers "F.Cu" "F.Mask" "F.Paste") (roundrect_rratio 0.25)
   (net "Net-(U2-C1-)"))
  (pad "11" smd roundrect (at 1.8625 -0.325 270) (size 1.025 0.35) (layers "F.Cu" "F.Mask" "F.Paste") (roundrect_rratio 0.25)
   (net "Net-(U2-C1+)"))
  (pad "12" smd roundrect (at 1.8625 -0.975 270) (size 1.025 0.35) (layers "F.Cu" "F.Mask" "F.Paste") (roundrect_rratio 0.25)
   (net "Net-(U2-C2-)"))
  (pad "13" smd roundrect (at 0.975 -1.8625 270) (size 0.35 1.025) (layers "F.Cu" "F.Mask" "F.Paste") (roundrect_rratio 0.25) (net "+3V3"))
  (pad "14" smd roundrect (at 0.325 -1.8625 270) (size 0.35 1.025) (layers "F.Cu" "F.Mask" "F.Paste") (roundrect_rratio 0.25) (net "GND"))
  (pad "15" smd roundrect (at -0.325 -1.8625 270) (size 0.35 1.025) (layers "F.Cu" "F.Mask" "F.Paste") (roundrect_rratio 0.25)
   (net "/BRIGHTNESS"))
  (pad "16" smd roundrect (at -0.975 -1.8625 270) (size 0.35 1.025) (layers "F.Cu" "F.Mask" "F.Paste") (roundrect_rratio 0.25)
   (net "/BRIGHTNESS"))
  (pad "17" smd rect (at 0 0 270) (size 2.1 2.1) (layers "F.Cu" "F.Mask") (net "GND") (zone_connect 2)))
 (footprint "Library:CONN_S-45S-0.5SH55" (layer "F.Cu") (at 45 10)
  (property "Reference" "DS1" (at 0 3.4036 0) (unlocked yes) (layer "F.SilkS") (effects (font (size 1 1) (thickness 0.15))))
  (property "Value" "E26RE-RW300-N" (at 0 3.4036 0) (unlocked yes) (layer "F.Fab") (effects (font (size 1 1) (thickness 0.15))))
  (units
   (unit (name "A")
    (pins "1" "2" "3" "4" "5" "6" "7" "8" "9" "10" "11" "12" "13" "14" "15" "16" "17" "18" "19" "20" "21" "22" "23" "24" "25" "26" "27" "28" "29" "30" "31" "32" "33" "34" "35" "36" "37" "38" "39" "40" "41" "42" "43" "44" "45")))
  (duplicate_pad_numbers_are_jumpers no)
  (fp_line (start -12.9286 -3.0734) (end -12.9286 -1.584841) (stroke (width 0.1524) (type solid)) (layer "F.SilkS"))
  (fp_line (start -12.9286 1.488539) (end -12.9286 3.0734) (stroke (width 0.1524) (type solid)) (layer "F.SilkS"))
  (fp_line (start -12.9286 3.0734) (end -11.497841 3.0734) (stroke (width 0.1524) (type solid)) (layer "F.SilkS"))
  (fp_line (start 11.497838 3.0734) (end 12.9286 3.0734) (stroke (width 0.1524) (type solid)) (layer "F.SilkS"))
  (fp_line (start 12.9286 -3.0734) (end -12.9286 -3.0734) (stroke (width 0.1524) (type solid)) (layer "F.SilkS"))
  (fp_line (start 12.9286 -1.584841) (end 12.9286 -3.0734) (stroke (width 0.1524) (type solid)) (layer "F.SilkS"))
  (fp_line (start 12.9286 3.0734) (end 12.9286 1.488539) (stroke (width 0.1524) (type solid)) (layer "F.SilkS"))
  (fp_circle (center -13.5636 3.4036) (end -13.1826 3.4036) (stroke (width 0.508) (type solid)) (fill no) (layer "F.SilkS"))
  (pad "1" smd rect (at -11.000001 3.1461) (size 0.3302 1.397) (layers "F.Cu" "F.Mask" "F.Paste") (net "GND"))
  (pad "2" smd rect (at -10.500002 3.1461) (size 0.3302 1.397) (layers "F.Cu" "F.Mask" "F.Paste") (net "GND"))
  (pad "3" smd rect (at -10 3.1461) (size 0.3302 1.397) (layers "F.Cu" "F.Mask" "F.Paste") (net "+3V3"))
  (pad "4" smd rect (at -9.500001 3.1461) (size 0.3302 1.397) (layers "F.Cu" "F.Mask" "F.Paste") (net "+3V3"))
  (pad "5" smd rect (at -9 3.1461) (size 0.3302 1.397) (layers "F.Cu" "F.Mask" "F.Paste") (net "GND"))
  (pad "6" smd rect (at -8.500001 3.1461) (size 0.3302 1.397) (layers "F.Cu" "F.Mask" "F.Paste") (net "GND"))
  (pad "7" smd rect (at -8.000002 3.1461) (size 0.3302 1.397) (layers "F.Cu" "F.Mask" "F.Paste") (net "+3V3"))
  (pad "8" smd rect (at -7.5 3.1461) (size 0.3302 1.397) (layers "F.Cu" "F.Mask" "F.Paste") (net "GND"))
  (pad "9" smd rect (at -7.000001 3.1461) (size 0.3302 1.397) (layers "F.Cu" "F.Mask" "F.Paste") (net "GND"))
  (pad "10" smd rect (at -6.5 3.1461) (size 0.3302 1.397) (layers "F.Cu" "F.Mask" "F.Paste") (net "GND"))
  (pad "11" smd rect (at -6.000001 3.1461) (size 0.3302 1.397) (layers "F.Cu" "F.Mask" "F.Paste") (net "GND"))
  (pad "12" smd rect (at -5.500002 3.1461) (size 0.3302 1.397) (layers "F.Cu" "F.Mask" "F.Paste") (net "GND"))
  (pad "13" smd rect (at -5 3.1461) (size 0.3302 1.397) (layers "F.Cu" "F.Mask" "F.Paste") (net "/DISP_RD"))
  (pad "14" smd rect (at -4.500001 3.1461) (size 0.3302 1.397) (layers "F.Cu" "F.Mask" "F.Paste") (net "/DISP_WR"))
  (pad "15" smd rect (at -4 3.1461) (size 0.3302 1.397) (layers "F.Cu" "F.Mask" "F.Paste") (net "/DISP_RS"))
  (pad "16" smd rect (at -3.500001 3.1461) (size 0.3302 1.397) (layers "F.Cu" "F.Mask" "F.Paste") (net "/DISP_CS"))
  (pad "17" smd rect (at -3.000002 3.1461) (size 0.3302 1.397) (layers "F.Cu" "F.Mask" "F.Paste") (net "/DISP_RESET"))
  (pad "18" smd rect (at -2.5 3.1461) (size 0.3302 1.397) (layers "F.Cu" "F.Mask" "F.Paste") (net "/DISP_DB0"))
  (pad "19" smd rect (at -2.000001 3.1461) (size 0.3302 1.397) (layers "F.Cu" "F.Mask" "F.Paste") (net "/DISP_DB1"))
  (pad "20" smd rect (at -1.5 3.1461) (size 0.3302 1.397) (layers "F.Cu" "F.Mask" "F.Paste") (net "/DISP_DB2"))
  (pad "21" smd rect (at -1.000001 3.1461) (size 0.3302 1.397) (layers "F.Cu" "F.Mask" "F.Paste") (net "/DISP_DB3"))
  (pad "22" smd rect (at -0.500002 3.1461) (size 0.3302 1.397) (layers "F.Cu" "F.Mask" "F.Paste") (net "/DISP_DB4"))
  (pad "23" smd rect (at 0 3.1461) (size 0.3302 1.397) (layers "F.Cu" "F.Mask" "F.Paste") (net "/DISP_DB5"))
  (pad "24" smd rect (at 0.499999 3.1461) (size 0.3302 1.397) (layers "F.Cu" "F.Mask" "F.Paste") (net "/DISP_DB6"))
  (pad "25" smd rect (at 1.000001 3.1461) (size 0.3302 1.397) (layers "F.Cu" "F.Mask" "F.Paste") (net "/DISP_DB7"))
  (pad "26" smd rect (at 1.5 3.1461) (size 0.3302 1.397) (layers "F.Cu" "F.Mask" "F.Paste") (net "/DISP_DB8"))
  (pad "27" smd rect (at 1.999999 3.1461) (size 0.3302 1.397) (layers "F.Cu" "F.Mask" "F.Paste") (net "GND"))
  (pad "28" smd rect (at 2.5 3.1461) (size 0.3302 1.397) (layers "F.Cu" "F.Mask" "F.Paste") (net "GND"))
  (pad "29" smd rect (at 2.999999 3.1461) (size 0.3302 1.397) (layers "F.Cu" "F.Mask" "F.Paste") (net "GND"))
  (pad "30" smd rect (at 3.500001 3.1461) (size 0.3302 1.397) (layers "F.Cu" "F.Mask" "F.Paste") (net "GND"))
  (pad "31" smd rect (at 4 3.1461) (size 0.3302 1.397) (layers "F.Cu" "F.Mask" "F.Paste") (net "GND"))
  (pad "32" smd rect (at 4.499999 3.1461) (size 0.3302 1.397) (layers "F.Cu" "F.Mask" "F.Paste") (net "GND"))
  (pad "33" smd rect (at 5 3.1461) (size 0.3302 1.397) (layers "F.Cu" "F.Mask" "F.Paste") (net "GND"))
  (pad "34" smd rect (at 5.499999 3.1461) (size 0.3302 1.397) (layers "F.Cu" "F.Mask" "F.Paste") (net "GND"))
  (pad "35" smd rect (at 6.000001 3.1461) (size 0.3302 1.397) (layers "F.Cu" "F.Mask" "F.Paste") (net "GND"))
  (pad "36" smd rect (at 6.5 3.1461) (size 0.3302 1.397) (layers "F.Cu" "F.Mask" "F.Paste") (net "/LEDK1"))
  (pad "37" smd rect (at 6.999999 3.1461) (size 0.3302 1.397) (layers "F.Cu" "F.Mask" "F.Paste") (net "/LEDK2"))
  (pad "38" smd rect (at 7.5 3.1461) (size 0.3302 1.397) (layers "F.Cu" "F.Mask" "F.Paste") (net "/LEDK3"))
  (pad "39" smd rect (at 7.999999 3.1461) (size 0.3302 1.397) (layers "F.Cu" "F.Mask" "F.Paste") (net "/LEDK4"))
  (pad "40" smd rect (at 8.499998 3.1461) (size 0.3302 1.397) (layers "F.Cu" "F.Mask" "F.Paste") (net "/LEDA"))
  (pad "41" smd rect (at 9 3.1461) (size 0.3302 1.397) (layers "F.Cu" "F.Mask" "F.Paste") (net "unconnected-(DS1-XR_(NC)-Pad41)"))
  (pad "42" smd rect (at 9.499999 3.1461) (size 0.3302 1.397) (layers "F.Cu" "F.Mask" "F.Paste") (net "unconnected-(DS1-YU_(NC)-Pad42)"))
  (pad "43" smd rect (at 10 3.1461) (size 0.3302 1.397) (layers "F.Cu" "F.Mask" "F.Paste") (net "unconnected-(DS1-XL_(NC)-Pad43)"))
  (pad "44" smd rect (at 10.499999 3.1461) (size 0.3302 1.397) (layers "F.Cu" "F.Mask" "F.Paste") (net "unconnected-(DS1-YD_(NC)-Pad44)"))
  (pad "45" smd rect (at 10.999998 3.1461) (size 0.3302 1.397) (layers "F.Cu" "F.Mask" "F.Paste") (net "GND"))
  (pad "46" smd rect (at -12.899999 0) (size 1.8034 2.3114) (layers "F.Cu" "F.Mask" "F.Paste"))
  (pad "47" smd rect (at 12.899999 0) (size 1.8034 2.3114) (layers "F.Cu" "F.Mask" "F.Paste")))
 (gr_rect (start 0 0) (end 90 100) (stroke (width 0.2) (type default)) (fill no) (layer "Edge.Cuts"))
 (segment (start 52.717529 15.417529) (end 60.862498 15.417529) (width 0.2) (layer "F.Cu") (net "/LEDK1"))
 (segment (start 51.5 13.105029) (end 51.5 14.2) (width 0.2) (layer "F.Cu") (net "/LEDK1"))
 (segment (start 51.5 14.2) (end 52.717529 15.417529) (width 0.2) (layer "F.Cu") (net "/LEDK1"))
 (segment (start 60.862498 16.067529) (end 62.399998 16.067529) (width 0.2) (layer "F.Cu") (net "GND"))
 (segment (start 64.587498 16.067529) (end 63.049998 16.067529) (width 0.2) (layer "F.Cu") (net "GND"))
 (segment (start 62.399998 16.067529) (end 62.724998 15.742529) (width 0.2) (layer "F.Cu") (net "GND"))
 (segment (start 63.049998 16.067529) (end 62.724998 15.742529) (width 0.2) (layer "F.Cu") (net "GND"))
 (segment (start 57.885372 14.767529) (end 58.060373 14.942529) (width 0.2) (layer "F.Cu") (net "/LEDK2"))
 (segment (start 60.687498 14.942529) (end 60.862498 14.767529) (width 0.2) (layer "F.Cu") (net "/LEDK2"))
 (segment (start 51.999999 14.134314) (end 52.633214 14.767529) (width 0.2) (layer "F.Cu") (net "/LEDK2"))
 (segment (start 52.633214 14.767529) (end 57.885372 14.767529) (width 0.2) (layer "F.Cu") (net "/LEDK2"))
 (segment (start 51.999999 13.105029) (end 51.999999 14.134314) (width 0.2) (layer "F.Cu") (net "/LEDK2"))
 (segment (start 58.060373 14.942529) (end 60.687498 14.942529) (width 0.2) (layer "F.Cu") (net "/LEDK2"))
 (segment (start 53.499998 13.105029) (end 53.499998 12.141431) (width 0.2) (layer "F.Cu") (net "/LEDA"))
 (segment (start 57.201498 12.106529) (end 58.357797 13.262828) (width 0.2) (layer "F.Cu") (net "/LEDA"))
 (segment (start 59.317529 16.717529) (end 59.3 16.7) (width 0.2) (layer "F.Cu") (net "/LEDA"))
 (segment (start 53.499998 12.141431) (end 53.5349 12.106529) (width 0.2) (layer "F.Cu") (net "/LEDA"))
 (segment (start 53.5349 12.106529) (end 57.201498 12.106529) (width 0.2) (layer "F.Cu") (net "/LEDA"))
 (segment (start 58.357797 13.262828) (end 58.357797 13.755029) (width 0.2) (layer "F.Cu") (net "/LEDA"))
 (segment (start 60.862498 16.717529) (end 59.317529 16.717529) (width 0.2) (layer "F.Cu") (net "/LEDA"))
 (via (at 59.3 16.7) (size 0.6) (drill 0.3) (layers "F.Cu" "B.Cu") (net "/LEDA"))
 (via (at 58.357797 13.755029) (size 0.6) (drill 0.3) (layers "F.Cu" "B.Cu") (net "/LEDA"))
 (segment (start 58.794969 16.7) (end 59.3 16.7) (width 0.2) (layer "B.Cu") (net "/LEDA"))
 (segment (start 58.357797 13.755029) (end 58.357797 16.262828) (width 0.2) (layer "B.Cu") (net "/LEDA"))
 (segment (start 58.357797 16.262828) (end 58.794969 16.7) (width 0.2) (layer "B.Cu") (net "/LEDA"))
 (segment (start 61.138997 12.106529) (end 62.399998 13.36753) (width 0.2) (layer "F.Cu") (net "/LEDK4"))
 (segment (start 62.399998 13.36753) (end 62.399998 13.880029) (width 0.2) (layer "F.Cu") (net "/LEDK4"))
 (segment (start 57.367184 11.706529) (end 57.767184 12.106529) (width 0.2) (layer "F.Cu") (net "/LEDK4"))
 (segment (start 57.767184 12.106529) (end 61.138997 12.106529) (width 0.2) (layer "F.Cu") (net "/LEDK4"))
 (segment (start 52.999999 13.105029) (end 52.999999 12.075745) (width 0.2) (layer "F.Cu") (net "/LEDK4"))
 (segment (start 53.369215 11.706529) (end 57.367184 11.706529) (width 0.2) (layer "F.Cu") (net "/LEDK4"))
 (segment (start 52.999999 12.075745) (end 53.369215 11.706529) (width 0.2) (layer "F.Cu") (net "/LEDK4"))
 (segment (start 52.5 14.06863) (end 52.534899 14.103529) (width 0.2) (layer "F.Cu") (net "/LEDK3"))
 (segment (start 59.152036 13.880029) (end 61.749998 13.880029) (width 0.2) (layer "F.Cu") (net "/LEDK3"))
 (segment (start 58.088558 14.405029) (end 58.627036 14.405029) (width 0.2) (layer "F.Cu") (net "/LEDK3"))
 (segment (start 58.627036 14.405029) (end 59.152036 13.880029) (width 0.2) (layer "F.Cu") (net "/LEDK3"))
 (segment (start 52.5 13.105029) (end 52.5 14.06863) (width 0.2) (layer "F.Cu") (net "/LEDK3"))
 (segment (start 57.787058 14.103529) (end 58.088558 14.405029) (width 0.2) (layer "F.Cu") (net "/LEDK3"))
 (segment (start 52.534899 14.103529) (end 57.787058 14.103529) (width 0.2) (layer "F.Cu") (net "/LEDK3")))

